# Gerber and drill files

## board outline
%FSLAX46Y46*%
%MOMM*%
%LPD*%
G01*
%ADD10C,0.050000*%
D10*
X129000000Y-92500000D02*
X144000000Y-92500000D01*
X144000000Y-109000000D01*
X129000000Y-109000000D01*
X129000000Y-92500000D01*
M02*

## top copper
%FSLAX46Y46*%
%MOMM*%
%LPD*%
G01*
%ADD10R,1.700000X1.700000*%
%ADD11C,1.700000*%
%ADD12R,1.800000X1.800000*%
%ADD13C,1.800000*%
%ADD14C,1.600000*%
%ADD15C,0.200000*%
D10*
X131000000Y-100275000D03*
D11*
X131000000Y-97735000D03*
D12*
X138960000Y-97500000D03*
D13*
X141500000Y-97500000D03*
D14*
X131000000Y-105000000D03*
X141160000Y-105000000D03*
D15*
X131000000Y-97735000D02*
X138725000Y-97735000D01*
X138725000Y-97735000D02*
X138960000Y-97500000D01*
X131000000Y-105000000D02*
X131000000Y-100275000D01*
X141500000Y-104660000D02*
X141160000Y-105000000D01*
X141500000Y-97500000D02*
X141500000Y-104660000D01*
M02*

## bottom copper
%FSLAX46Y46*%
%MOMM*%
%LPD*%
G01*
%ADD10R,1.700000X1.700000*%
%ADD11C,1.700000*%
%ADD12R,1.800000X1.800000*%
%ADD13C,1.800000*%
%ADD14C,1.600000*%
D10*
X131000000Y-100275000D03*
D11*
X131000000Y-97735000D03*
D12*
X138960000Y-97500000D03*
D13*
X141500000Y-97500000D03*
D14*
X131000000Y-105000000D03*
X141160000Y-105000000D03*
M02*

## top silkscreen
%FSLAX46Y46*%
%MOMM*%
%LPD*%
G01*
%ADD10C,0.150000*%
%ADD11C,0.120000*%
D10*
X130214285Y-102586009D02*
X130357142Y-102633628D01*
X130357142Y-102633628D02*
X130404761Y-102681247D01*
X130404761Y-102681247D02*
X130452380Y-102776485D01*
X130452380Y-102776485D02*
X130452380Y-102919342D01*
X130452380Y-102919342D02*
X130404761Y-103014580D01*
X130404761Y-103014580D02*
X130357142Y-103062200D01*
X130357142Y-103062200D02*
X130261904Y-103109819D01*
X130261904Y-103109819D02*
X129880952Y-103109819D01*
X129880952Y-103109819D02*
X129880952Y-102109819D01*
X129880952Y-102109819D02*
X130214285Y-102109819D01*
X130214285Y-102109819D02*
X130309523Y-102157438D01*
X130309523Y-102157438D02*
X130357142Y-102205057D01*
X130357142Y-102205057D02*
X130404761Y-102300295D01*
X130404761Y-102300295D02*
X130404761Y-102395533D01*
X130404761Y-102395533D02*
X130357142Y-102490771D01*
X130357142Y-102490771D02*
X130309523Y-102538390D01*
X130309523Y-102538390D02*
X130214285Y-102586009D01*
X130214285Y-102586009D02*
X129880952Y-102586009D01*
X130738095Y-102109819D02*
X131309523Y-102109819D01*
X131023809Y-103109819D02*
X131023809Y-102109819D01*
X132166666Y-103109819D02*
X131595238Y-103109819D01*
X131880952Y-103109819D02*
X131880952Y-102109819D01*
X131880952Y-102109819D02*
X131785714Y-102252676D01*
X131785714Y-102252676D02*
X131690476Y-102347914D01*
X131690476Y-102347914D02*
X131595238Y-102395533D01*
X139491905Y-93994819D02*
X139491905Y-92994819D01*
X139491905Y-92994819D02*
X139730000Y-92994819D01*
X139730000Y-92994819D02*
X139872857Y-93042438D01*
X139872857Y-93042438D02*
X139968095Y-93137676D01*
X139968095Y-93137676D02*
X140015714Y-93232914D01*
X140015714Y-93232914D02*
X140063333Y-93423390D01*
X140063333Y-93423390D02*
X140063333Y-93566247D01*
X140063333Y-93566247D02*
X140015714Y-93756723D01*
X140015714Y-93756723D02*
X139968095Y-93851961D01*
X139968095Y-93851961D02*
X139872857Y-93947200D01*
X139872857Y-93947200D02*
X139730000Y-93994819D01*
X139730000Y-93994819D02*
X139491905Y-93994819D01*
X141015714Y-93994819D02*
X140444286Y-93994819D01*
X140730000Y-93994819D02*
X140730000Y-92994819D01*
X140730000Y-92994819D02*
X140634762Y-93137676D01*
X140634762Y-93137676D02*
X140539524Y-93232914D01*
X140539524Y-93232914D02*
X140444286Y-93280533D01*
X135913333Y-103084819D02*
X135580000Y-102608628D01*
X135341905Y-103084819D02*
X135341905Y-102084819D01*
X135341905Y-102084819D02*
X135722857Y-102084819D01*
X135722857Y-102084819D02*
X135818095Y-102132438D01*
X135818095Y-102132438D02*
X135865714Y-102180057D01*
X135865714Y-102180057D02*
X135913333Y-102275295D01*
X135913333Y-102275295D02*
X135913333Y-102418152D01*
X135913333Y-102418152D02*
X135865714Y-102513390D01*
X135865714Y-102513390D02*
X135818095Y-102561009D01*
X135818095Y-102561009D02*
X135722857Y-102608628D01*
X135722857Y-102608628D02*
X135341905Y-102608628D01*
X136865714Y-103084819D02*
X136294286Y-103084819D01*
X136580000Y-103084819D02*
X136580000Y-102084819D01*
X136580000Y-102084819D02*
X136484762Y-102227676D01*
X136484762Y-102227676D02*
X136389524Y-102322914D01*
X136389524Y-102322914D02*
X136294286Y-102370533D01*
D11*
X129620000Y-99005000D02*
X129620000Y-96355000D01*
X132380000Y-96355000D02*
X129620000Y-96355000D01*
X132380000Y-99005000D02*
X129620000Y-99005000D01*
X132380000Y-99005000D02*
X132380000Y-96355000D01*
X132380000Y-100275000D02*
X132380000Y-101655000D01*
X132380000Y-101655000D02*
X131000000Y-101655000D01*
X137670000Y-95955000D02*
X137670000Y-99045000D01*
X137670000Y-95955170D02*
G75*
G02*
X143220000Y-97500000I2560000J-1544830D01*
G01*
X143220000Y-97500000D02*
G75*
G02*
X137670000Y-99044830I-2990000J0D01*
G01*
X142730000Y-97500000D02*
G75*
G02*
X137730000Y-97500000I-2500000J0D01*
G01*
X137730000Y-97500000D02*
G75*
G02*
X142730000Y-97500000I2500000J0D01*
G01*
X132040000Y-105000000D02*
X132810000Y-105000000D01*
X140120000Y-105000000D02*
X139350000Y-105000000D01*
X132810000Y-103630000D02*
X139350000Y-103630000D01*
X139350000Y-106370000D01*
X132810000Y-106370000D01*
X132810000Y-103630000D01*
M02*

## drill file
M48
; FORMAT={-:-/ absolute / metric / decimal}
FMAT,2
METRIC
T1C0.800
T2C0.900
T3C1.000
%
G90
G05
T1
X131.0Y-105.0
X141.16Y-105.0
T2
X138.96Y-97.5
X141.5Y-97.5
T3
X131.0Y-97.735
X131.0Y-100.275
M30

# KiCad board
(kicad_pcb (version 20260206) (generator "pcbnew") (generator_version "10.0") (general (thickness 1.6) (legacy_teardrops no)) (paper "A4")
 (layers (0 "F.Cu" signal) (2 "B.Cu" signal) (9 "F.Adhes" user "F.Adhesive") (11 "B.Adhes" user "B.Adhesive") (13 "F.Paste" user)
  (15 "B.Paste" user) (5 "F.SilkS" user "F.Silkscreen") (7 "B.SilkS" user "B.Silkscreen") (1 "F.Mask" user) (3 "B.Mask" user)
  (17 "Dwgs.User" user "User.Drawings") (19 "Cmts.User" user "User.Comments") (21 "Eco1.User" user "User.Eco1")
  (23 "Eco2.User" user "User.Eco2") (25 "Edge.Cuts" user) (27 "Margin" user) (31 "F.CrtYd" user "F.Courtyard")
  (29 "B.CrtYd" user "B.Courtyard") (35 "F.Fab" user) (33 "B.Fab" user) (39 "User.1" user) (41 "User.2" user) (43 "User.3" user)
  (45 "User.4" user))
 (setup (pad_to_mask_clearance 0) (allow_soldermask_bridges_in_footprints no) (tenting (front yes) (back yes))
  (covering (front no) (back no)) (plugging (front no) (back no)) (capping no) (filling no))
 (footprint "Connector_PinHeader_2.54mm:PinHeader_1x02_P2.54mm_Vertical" (layer "F.Cu") (at 131 100.275 180)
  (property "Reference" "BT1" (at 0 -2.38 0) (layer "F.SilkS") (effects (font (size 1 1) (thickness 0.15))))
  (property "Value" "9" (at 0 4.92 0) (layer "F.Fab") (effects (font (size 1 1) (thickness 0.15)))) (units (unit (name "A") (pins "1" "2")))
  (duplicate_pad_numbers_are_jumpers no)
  (fp_line (start 1.38 1.27) (end 1.38 3.92) (stroke (width 0.12) (type solid)) (layer "F.SilkS"))
  (fp_line (start -1.38 3.92) (end 1.38 3.92) (stroke (width 0.12) (type solid)) (layer "F.SilkS"))
  (fp_line (start -1.38 1.27) (end 1.38 1.27) (stroke (width 0.12) (type solid)) (layer "F.SilkS"))
  (fp_line (start -1.38 1.27) (end -1.38 3.92) (stroke (width 0.12) (type solid)) (layer "F.SilkS"))
  (fp_line (start -1.38 0) (end -1.38 -1.38) (stroke (width 0.12) (type solid)) (layer "F.SilkS"))
  (fp_line (start -1.38 -1.38) (end 0 -1.38) (stroke (width 0.12) (type solid)) (layer "F.SilkS"))
  (pad "1" thru_hole rect (at 0 0 180) (size 1.7 1.7) (drill 1) (layers "*.Cu" "*.Mask") (remove_unused_layers no) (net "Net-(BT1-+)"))
  (pad "2" thru_hole circle (at 0 2.54 180) (size 1.7 1.7) (drill 1) (layers "*.Cu" "*.Mask") (remove_unused_layers no) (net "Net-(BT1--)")))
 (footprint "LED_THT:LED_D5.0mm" (layer "F.Cu") (at 138.96 97.5)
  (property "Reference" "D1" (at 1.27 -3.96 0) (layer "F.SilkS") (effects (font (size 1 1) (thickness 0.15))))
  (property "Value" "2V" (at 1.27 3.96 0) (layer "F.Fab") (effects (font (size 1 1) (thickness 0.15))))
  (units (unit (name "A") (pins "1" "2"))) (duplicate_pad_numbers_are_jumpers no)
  (fp_line (start -1.29 -1.545) (end -1.29 1.545) (stroke (width 0.12) (type solid)) (layer "F.SilkS"))
  (fp_arc (start -1.29 -1.54483) (mid 2.071779 -2.880495) (end 4.26 0) (stroke (width 0.12) (type solid)) (layer "F.SilkS"))
  (fp_arc (start 4.26 0) (mid 2.071779 2.880495) (end -1.29 1.54483) (stroke (width 0.12) (type solid)) (layer "F.SilkS"))
  (fp_circle (center 1.27 0) (end 3.77 0) (stroke (width 0.12) (type solid)) (fill no) (layer "F.SilkS"))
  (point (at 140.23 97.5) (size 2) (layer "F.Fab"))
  (pad "1" thru_hole rect (at 0 0) (size 1.8 1.8) (drill 0.9) (layers "*.Cu" "*.Mask") (remove_unused_layers no) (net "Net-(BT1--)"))
  (pad "2" thru_hole circle (at 2.54 0) (size 1.8 1.8) (drill 0.9) (layers "*.Cu" "*.Mask") (remove_unused_layers no) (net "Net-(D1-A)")))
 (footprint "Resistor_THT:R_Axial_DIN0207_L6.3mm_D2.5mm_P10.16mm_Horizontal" (layer "F.Cu") (at 131 105)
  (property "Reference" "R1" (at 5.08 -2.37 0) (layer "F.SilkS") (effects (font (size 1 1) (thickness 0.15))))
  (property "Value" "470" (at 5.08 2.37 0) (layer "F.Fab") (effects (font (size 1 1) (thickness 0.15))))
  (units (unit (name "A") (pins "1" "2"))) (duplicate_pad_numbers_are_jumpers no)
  (fp_line (start 1.04 0) (end 1.81 0) (stroke (width 0.12) (type solid)) (layer "F.SilkS"))
  (fp_line (start 9.12 0) (end 8.35 0) (stroke (width 0.12) (type solid)) (layer "F.SilkS"))
  (fp_rect (start 1.81 -1.37) (end 8.35 1.37) (stroke (width 0.12) (type solid)) (fill no) (layer "F.SilkS"))
  (pad "1" thru_hole circle (at 0 0) (size 1.6 1.6) (drill 0.8) (layers "*.Cu" "*.Mask") (remove_unused_layers no) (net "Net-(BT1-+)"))
  (pad "2" thru_hole circle (at 10.16 0) (size 1.6 1.6) (drill 0.8) (layers "*.Cu" "*.Mask") (remove_unused_layers no) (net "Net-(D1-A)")))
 (gr_poly (pts (xy 129 92.5) (xy 144 92.5) (xy 144 109) (xy 129 109)) (stroke (width 0.05) (type solid)) (fill no) (layer "Edge.Cuts"))
 (segment (start 131 97.735) (end 138.725 97.735) (width 0.2) (layer "F.Cu") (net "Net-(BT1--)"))
 (segment (start 138.725 97.735) (end 138.96 97.5) (width 0.2) (layer "F.Cu") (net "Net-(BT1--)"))
 (segment (start 131 105) (end 131 100.275) (width 0.2) (layer "F.Cu") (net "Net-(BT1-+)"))
 (segment (start 141.5 104.66) (end 141.16 105) (width 0.2) (layer "F.Cu") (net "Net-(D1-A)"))
 (segment (start 141.5 97.5) (end 141.5 104.66) (width 0.2) (layer "F.Cu") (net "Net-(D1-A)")))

